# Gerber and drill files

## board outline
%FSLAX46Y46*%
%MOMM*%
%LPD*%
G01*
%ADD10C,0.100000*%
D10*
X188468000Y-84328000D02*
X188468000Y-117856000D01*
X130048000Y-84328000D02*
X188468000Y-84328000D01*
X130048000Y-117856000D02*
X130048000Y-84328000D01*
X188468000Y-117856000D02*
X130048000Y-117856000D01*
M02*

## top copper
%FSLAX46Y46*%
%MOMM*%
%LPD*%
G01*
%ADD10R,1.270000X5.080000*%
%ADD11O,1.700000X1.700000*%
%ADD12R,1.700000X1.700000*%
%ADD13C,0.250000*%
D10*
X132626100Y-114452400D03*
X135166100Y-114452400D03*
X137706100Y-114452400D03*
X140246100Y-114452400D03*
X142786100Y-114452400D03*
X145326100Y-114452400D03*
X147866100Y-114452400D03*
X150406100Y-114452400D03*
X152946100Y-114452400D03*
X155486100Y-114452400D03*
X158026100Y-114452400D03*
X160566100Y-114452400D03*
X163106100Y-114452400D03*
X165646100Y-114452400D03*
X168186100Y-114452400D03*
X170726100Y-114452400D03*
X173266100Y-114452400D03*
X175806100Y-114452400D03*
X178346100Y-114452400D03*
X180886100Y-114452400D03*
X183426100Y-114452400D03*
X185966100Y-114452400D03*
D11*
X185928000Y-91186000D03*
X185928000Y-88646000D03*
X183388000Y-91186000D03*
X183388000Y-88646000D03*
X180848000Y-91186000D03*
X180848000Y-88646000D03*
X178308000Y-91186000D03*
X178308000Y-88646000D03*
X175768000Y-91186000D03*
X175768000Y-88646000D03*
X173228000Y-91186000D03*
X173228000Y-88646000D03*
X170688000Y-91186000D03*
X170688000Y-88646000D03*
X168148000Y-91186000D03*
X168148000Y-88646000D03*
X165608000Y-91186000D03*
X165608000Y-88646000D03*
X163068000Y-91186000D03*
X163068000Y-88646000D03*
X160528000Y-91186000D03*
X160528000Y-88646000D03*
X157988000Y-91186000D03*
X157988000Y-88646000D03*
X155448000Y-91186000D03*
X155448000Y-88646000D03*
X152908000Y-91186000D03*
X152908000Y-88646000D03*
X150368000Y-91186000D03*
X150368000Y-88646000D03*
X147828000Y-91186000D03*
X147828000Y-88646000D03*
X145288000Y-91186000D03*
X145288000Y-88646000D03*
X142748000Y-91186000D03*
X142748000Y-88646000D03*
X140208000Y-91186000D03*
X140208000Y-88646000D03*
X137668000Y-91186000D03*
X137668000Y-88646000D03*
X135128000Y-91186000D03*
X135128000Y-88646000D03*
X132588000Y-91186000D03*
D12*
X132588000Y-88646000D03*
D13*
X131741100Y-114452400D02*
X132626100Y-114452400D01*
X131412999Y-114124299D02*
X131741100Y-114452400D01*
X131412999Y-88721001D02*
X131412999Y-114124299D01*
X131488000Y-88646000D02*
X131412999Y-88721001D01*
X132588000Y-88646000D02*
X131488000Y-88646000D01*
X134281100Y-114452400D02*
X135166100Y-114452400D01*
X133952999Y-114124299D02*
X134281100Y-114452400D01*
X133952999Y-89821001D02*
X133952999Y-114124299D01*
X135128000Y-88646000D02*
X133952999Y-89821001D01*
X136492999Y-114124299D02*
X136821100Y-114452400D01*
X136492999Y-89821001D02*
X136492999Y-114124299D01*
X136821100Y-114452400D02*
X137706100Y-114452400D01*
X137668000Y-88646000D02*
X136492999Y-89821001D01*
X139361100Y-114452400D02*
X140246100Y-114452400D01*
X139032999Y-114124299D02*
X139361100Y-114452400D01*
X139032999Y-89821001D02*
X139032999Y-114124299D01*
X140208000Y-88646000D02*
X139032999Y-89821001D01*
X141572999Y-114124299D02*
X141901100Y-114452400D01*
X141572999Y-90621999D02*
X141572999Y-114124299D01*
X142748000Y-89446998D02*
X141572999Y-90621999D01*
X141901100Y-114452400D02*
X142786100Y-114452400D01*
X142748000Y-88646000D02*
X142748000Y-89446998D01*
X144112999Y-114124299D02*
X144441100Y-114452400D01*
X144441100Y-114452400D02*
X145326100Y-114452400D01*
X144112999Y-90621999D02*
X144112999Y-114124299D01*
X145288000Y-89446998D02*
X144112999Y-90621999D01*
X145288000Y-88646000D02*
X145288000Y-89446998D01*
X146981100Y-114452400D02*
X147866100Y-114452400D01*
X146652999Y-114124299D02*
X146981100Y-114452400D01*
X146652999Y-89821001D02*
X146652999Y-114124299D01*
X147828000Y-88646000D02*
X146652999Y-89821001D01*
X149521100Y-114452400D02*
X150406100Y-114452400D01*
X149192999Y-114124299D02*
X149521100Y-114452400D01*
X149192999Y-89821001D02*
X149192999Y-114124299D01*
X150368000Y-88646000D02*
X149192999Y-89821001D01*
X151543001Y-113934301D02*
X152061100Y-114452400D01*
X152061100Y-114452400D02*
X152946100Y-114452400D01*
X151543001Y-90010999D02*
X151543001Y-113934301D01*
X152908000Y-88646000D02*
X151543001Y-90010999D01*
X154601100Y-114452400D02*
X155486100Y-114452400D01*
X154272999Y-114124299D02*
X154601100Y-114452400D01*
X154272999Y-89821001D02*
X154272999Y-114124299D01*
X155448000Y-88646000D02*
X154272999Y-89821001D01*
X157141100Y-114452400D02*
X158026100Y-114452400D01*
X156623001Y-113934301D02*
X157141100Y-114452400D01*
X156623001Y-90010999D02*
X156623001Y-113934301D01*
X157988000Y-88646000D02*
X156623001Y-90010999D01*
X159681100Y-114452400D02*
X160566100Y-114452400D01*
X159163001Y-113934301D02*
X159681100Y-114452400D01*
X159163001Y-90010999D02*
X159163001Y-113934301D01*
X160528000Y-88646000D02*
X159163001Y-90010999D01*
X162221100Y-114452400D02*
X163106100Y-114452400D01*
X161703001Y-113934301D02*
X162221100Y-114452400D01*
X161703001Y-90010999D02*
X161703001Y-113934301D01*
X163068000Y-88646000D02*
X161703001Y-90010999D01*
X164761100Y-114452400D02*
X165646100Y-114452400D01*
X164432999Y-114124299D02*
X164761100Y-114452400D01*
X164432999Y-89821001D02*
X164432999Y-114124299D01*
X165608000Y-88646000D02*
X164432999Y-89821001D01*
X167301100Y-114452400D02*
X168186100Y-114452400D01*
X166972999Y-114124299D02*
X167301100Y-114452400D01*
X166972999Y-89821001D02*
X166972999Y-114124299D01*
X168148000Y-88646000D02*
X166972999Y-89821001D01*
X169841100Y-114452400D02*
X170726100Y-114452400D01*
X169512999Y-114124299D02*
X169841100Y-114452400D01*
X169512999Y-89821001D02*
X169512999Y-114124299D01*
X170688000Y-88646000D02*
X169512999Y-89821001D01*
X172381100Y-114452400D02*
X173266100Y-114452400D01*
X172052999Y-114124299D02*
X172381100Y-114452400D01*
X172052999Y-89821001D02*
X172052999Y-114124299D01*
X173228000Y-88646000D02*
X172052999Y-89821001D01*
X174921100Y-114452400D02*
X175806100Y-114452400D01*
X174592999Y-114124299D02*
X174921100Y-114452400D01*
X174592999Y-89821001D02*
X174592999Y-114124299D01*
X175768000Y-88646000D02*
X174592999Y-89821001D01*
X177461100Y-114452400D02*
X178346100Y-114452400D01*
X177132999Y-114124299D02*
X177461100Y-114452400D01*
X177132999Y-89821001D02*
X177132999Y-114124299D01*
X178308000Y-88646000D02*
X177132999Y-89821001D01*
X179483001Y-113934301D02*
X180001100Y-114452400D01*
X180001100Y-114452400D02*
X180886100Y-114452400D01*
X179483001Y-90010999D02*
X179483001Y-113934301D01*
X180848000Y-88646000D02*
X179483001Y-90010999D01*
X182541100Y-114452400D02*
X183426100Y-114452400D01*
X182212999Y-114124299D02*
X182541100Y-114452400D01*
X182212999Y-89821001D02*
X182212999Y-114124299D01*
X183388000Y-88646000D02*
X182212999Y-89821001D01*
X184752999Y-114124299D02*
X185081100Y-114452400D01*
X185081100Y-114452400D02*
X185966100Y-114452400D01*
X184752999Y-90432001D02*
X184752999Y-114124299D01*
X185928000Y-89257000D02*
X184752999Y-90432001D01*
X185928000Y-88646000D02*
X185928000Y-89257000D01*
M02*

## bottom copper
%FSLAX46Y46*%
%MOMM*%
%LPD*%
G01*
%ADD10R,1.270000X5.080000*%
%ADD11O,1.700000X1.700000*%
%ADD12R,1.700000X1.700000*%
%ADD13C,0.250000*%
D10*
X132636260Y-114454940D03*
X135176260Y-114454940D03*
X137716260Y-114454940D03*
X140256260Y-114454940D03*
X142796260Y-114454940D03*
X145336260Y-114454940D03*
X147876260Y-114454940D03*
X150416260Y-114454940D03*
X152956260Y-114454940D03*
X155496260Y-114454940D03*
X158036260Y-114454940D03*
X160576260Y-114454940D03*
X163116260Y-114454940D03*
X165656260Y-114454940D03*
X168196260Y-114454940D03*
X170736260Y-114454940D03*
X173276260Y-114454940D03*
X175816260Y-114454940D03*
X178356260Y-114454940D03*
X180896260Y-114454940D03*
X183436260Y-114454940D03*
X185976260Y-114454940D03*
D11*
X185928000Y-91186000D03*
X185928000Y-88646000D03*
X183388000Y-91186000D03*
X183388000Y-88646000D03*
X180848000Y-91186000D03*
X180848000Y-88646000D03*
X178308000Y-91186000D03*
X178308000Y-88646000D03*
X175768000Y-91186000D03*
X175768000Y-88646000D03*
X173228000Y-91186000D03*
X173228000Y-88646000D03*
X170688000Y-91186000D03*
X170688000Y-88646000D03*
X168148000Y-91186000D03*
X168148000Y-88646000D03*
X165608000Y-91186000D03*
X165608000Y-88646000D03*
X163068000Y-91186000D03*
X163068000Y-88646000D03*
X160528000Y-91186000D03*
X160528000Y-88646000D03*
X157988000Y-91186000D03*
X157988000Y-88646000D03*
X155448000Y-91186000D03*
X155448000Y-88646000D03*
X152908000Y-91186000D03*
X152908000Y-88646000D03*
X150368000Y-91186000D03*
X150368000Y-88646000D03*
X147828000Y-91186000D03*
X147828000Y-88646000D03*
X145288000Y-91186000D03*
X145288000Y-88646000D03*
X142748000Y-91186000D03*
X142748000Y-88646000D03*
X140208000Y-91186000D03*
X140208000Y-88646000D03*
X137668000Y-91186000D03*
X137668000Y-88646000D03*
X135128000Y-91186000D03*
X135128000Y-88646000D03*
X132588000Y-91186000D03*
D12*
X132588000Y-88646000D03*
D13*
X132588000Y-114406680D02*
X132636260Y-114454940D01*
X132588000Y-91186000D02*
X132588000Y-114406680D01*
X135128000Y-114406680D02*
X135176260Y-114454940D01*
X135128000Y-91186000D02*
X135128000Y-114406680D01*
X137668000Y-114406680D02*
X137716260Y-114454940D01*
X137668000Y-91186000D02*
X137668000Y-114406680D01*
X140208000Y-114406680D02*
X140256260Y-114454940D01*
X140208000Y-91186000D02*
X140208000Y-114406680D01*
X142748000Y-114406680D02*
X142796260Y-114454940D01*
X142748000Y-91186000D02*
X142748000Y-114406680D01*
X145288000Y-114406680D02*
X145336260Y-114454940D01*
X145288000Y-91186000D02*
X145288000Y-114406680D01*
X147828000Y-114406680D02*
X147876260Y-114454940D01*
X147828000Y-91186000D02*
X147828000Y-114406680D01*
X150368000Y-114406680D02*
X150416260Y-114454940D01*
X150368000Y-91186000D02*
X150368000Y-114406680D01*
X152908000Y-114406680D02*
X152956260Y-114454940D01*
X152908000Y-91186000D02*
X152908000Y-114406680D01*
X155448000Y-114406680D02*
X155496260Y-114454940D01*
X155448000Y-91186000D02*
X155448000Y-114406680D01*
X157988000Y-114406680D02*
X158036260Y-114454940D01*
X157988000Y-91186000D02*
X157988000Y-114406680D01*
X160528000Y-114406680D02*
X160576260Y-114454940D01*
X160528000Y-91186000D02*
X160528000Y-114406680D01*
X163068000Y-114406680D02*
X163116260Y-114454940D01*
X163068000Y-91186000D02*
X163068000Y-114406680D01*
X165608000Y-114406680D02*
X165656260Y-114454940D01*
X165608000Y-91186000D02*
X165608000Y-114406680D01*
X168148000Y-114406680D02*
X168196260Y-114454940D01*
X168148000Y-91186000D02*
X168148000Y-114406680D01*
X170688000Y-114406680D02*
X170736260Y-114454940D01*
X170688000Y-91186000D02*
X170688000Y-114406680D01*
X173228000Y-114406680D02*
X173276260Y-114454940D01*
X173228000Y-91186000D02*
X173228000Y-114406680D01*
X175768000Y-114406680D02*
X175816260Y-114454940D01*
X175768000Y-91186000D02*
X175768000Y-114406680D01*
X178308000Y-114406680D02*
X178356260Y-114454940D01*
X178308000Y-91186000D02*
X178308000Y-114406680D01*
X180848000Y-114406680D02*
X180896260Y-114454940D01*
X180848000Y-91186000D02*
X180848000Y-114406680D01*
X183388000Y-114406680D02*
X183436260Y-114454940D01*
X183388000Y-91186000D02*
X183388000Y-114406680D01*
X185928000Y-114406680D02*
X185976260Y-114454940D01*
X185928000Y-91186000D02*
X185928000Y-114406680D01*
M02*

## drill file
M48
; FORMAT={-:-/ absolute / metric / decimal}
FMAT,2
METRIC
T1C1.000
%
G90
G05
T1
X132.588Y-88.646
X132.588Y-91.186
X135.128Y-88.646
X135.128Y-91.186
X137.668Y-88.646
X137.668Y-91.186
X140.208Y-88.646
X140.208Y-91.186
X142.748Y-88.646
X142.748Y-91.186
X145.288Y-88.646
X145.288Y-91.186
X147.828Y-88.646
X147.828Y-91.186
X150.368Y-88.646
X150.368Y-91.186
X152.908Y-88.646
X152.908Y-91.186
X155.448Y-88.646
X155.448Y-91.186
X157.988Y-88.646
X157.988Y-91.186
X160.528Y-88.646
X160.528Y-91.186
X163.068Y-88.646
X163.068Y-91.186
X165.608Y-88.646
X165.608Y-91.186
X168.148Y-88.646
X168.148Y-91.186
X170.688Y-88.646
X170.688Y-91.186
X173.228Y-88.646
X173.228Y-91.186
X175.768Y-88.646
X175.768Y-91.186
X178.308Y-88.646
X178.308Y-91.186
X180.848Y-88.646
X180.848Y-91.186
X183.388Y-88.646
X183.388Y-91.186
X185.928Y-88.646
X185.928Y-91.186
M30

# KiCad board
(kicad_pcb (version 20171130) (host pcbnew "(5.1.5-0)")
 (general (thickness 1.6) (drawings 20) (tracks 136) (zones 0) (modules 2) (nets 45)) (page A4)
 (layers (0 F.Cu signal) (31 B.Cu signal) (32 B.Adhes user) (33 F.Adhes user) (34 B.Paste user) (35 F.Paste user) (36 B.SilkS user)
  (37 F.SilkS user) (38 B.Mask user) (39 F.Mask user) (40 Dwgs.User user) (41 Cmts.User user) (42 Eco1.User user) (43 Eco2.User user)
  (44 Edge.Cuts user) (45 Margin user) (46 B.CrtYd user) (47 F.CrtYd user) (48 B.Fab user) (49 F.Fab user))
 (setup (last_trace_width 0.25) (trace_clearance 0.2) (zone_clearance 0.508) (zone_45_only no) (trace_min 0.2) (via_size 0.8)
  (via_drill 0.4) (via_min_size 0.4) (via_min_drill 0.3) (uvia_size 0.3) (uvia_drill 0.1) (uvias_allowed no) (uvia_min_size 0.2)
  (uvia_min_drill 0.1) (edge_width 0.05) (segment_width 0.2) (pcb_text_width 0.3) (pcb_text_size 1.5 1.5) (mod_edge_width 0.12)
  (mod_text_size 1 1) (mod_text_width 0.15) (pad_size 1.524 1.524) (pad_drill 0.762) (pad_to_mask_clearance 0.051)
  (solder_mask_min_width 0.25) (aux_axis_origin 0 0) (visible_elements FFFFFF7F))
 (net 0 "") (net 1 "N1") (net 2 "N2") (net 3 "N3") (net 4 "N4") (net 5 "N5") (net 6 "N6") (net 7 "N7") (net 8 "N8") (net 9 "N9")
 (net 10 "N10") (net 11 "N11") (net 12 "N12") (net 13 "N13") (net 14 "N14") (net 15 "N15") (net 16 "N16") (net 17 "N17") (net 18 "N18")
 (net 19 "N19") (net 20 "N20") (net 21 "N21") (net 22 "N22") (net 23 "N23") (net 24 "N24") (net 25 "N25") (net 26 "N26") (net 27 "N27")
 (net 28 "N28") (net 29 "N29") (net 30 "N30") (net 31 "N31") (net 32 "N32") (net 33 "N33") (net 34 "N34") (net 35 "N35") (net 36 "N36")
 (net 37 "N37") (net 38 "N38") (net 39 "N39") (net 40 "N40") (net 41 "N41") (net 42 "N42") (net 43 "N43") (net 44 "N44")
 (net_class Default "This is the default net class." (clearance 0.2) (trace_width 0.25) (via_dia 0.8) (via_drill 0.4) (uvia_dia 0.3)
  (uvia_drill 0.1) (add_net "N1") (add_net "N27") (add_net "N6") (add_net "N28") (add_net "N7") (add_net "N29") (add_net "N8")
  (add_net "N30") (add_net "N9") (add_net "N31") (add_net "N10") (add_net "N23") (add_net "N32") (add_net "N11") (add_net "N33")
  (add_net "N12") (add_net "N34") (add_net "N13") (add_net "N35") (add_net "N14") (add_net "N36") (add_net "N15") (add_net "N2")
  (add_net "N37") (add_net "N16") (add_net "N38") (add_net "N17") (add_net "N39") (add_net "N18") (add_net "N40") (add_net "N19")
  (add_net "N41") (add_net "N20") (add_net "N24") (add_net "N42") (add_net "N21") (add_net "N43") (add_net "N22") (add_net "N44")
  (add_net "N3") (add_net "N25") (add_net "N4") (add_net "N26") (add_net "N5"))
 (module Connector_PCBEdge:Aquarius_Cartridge (layer F.Cu) (at 144.272 102.362)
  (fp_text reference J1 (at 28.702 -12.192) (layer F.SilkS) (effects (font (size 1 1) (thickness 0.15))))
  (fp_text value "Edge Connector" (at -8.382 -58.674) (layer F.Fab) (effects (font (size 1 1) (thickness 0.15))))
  (pad 1 connect rect (at -11.6459 12.0904) (size 1.27 5.08) (layers F.Cu F.Mask) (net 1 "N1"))
  (pad 3 connect rect (at -9.1059 12.0904) (size 1.27 5.08) (layers F.Cu F.Mask) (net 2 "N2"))
  (pad 5 connect rect (at -6.5659 12.0904) (size 1.27 5.08) (layers F.Cu F.Mask) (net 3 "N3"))
  (pad 7 connect rect (at -4.0259 12.0904) (size 1.27 5.08) (layers F.Cu F.Mask) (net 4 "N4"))
  (pad 9 connect rect (at -1.4859 12.0904) (size 1.27 5.08) (layers F.Cu F.Mask) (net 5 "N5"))
  (pad 11 connect rect (at 1.0541 12.0904) (size 1.27 5.08) (layers F.Cu F.Mask) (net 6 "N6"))
  (pad 13 connect rect (at 3.5941 12.0904) (size 1.27 5.08) (layers F.Cu F.Mask) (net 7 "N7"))
  (pad 15 connect rect (at 6.1341 12.0904) (size 1.27 5.08) (layers F.Cu F.Mask) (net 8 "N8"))
  (pad 17 connect rect (at 8.6741 12.0904) (size 1.27 5.08) (layers F.Cu F.Mask) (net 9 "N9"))
  (pad 19 connect rect (at 11.2141 12.0904) (size 1.27 5.08) (layers F.Cu F.Mask) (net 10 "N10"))
  (pad 21 connect rect (at 13.7541 12.0904) (size 1.27 5.08) (layers F.Cu F.Mask) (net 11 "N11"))
  (pad 23 connect rect (at 16.2941 12.0904) (size 1.27 5.08) (layers F.Cu F.Mask) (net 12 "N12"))
  (pad 25 connect rect (at 18.8341 12.0904) (size 1.27 5.08) (layers F.Cu F.Mask) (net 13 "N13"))
  (pad 27 connect rect (at 21.3741 12.0904) (size 1.27 5.08) (layers F.Cu F.Mask) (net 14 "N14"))
  (pad 29 connect rect (at 23.9141 12.0904) (size 1.27 5.08) (layers F.Cu F.Mask) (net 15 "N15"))
  (pad 31 connect rect (at 26.4541 12.0904) (size 1.27 5.08) (layers F.Cu F.Mask) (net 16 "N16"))
  (pad 33 connect rect (at 28.9941 12.0904) (size 1.27 5.08) (layers F.Cu F.Mask) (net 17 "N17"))
  (pad 35 connect rect (at 31.5341 12.0904) (size 1.27 5.08) (layers F.Cu F.Mask) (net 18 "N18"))
  (pad 37 connect rect (at 34.0741 12.0904) (size 1.27 5.08) (layers F.Cu F.Mask) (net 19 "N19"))
  (pad 39 connect rect (at 36.6141 12.0904) (size 1.27 5.08) (layers F.Cu F.Mask) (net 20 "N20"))
  (pad 41 connect rect (at 39.1541 12.0904) (size 1.27 5.08) (layers F.Cu F.Mask) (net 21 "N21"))
  (pad 43 connect rect (at 41.6941 12.0904) (size 1.27 5.08) (layers F.Cu F.Mask) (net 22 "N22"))
  (pad 2 connect rect (at -11.63574 12.09294) (size 1.27 5.08) (layers B.Cu B.Mask) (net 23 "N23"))
  (pad 4 connect rect (at -9.09574 12.09294) (size 1.27 5.08) (layers B.Cu B.Mask) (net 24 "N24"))
  (pad 6 connect rect (at -6.55574 12.09294) (size 1.27 5.08) (layers B.Cu B.Mask) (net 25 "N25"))
  (pad 8 connect rect (at -4.01574 12.09294) (size 1.27 5.08) (layers B.Cu B.Mask) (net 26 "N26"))
  (pad 10 connect rect (at -1.47574 12.09294) (size 1.27 5.08) (layers B.Cu B.Mask) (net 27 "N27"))
  (pad 12 connect rect (at 1.06426 12.09294) (size 1.27 5.08) (layers B.Cu B.Mask) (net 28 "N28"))
  (pad 14 connect rect (at 3.60426 12.09294) (size 1.27 5.08) (layers B.Cu B.Mask) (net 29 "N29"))
  (pad 16 connect rect (at 6.14426 12.09294) (size 1.27 5.08) (layers B.Cu B.Mask) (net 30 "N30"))
  (pad 18 connect rect (at 8.68426 12.09294) (size 1.27 5.08) (layers B.Cu B.Mask) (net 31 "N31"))
  (pad 20 connect rect (at 11.22426 12.09294) (size 1.27 5.08) (layers B.Cu B.Mask) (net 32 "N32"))
  (pad 22 connect rect (at 13.76426 12.09294) (size 1.27 5.08) (layers B.Cu B.Mask) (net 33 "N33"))
  (pad 24 connect rect (at 16.30426 12.09294) (size 1.27 5.08) (layers B.Cu B.Mask) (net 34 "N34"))
  (pad 26 connect rect (at 18.84426 12.09294) (size 1.27 5.08) (layers B.Cu B.Mask) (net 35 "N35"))
  (pad 28 connect rect (at 21.38426 12.09294) (size 1.27 5.08) (layers B.Cu B.Mask) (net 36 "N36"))
  (pad 30 connect rect (at 23.92426 12.09294) (size 1.27 5.08) (layers B.Cu B.Mask) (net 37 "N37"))
  (pad 32 connect rect (at 26.46426 12.09294) (size 1.27 5.08) (layers B.Cu B.Mask) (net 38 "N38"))
  (pad 34 connect rect (at 29.00426 12.09294) (size 1.27 5.08) (layers B.Cu B.Mask) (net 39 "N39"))
  (pad 36 connect rect (at 31.54426 12.09294) (size 1.27 5.08) (layers B.Cu B.Mask) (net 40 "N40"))
  (pad 38 connect rect (at 34.08426 12.09294) (size 1.27 5.08) (layers B.Cu B.Mask) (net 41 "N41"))
  (pad 40 connect rect (at 36.62426 12.09294) (size 1.27 5.08) (layers B.Cu B.Mask) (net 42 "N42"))
  (pad 42 connect rect (at 39.16426 12.09294) (size 1.27 5.08) (layers B.Cu B.Mask) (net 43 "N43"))
  (pad 44 connect rect (at 41.70426 12.09294) (size 1.27 5.08) (layers B.Cu B.Mask) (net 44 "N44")))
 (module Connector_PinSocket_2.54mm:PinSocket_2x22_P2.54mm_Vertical (layer F.Cu) (at 132.588 88.646 90)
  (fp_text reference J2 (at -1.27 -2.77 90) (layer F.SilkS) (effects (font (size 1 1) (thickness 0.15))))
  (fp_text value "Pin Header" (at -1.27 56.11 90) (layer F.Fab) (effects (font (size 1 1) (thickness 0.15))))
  (pad 44 thru_hole oval (at -2.54 53.34 90) (size 1.7 1.7) (drill 1) (layers *.Cu *.Mask) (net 44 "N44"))
  (pad 43 thru_hole oval (at 0 53.34 90) (size 1.7 1.7) (drill 1) (layers *.Cu *.Mask) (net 22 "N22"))
  (pad 42 thru_hole oval (at -2.54 50.8 90) (size 1.7 1.7) (drill 1) (layers *.Cu *.Mask) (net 43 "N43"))
  (pad 41 thru_hole oval (at 0 50.8 90) (size 1.7 1.7) (drill 1) (layers *.Cu *.Mask) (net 21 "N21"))
  (pad 40 thru_hole oval (at -2.54 48.26 90) (size 1.7 1.7) (drill 1) (layers *.Cu *.Mask) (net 42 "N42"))
  (pad 39 thru_hole oval (at 0 48.26 90) (size 1.7 1.7) (drill 1) (layers *.Cu *.Mask) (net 20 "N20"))
  (pad 38 thru_hole oval (at -2.54 45.72 90) (size 1.7 1.7) (drill 1) (layers *.Cu *.Mask) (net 41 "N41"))
  (pad 37 thru_hole oval (at 0 45.72 90) (size 1.7 1.7) (drill 1) (layers *.Cu *.Mask) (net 19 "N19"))
  (pad 36 thru_hole oval (at -2.54 43.18 90) (size 1.7 1.7) (drill 1) (layers *.Cu *.Mask) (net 40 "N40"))
  (pad 35 thru_hole oval (at 0 43.18 90) (size 1.7 1.7) (drill 1) (layers *.Cu *.Mask) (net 18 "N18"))
  (pad 34 thru_hole oval (at -2.54 40.64 90) (size 1.7 1.7) (drill 1) (layers *.Cu *.Mask) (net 39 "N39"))
  (pad 33 thru_hole oval (at 0 40.64 90) (size 1.7 1.7) (drill 1) (layers *.Cu *.Mask) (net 17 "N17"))
  (pad 32 thru_hole oval (at -2.54 38.1 90) (size 1.7 1.7) (drill 1) (layers *.Cu *.Mask) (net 38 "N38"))
  (pad 31 thru_hole oval (at 0 38.1 90) (size 1.7 1.7) (drill 1) (layers *.Cu *.Mask) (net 16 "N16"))
  (pad 30 thru_hole oval (at -2.54 35.56 90) (size 1.7 1.7) (drill 1) (layers *.Cu *.Mask) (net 37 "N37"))
  (pad 29 thru_hole oval (at 0 35.56 90) (size 1.7 1.7) (drill 1) (layers *.Cu *.Mask) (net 15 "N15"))
  (pad 28 thru_hole oval (at -2.54 33.02 90) (size 1.7 1.7) (drill 1) (layers *.Cu *.Mask) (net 36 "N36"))
  (pad 27 thru_hole oval (at 0 33.02 90) (size 1.7 1.7) (drill 1) (layers *.Cu *.Mask) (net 14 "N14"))
  (pad 26 thru_hole oval (at -2.54 30.48 90) (size 1.7 1.7) (drill 1) (layers *.Cu *.Mask) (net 35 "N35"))
  (pad 25 thru_hole oval (at 0 30.48 90) (size 1.7 1.7) (drill 1) (layers *.Cu *.Mask) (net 13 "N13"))
  (pad 24 thru_hole oval (at -2.54 27.94 90) (size 1.7 1.7) (drill 1) (layers *.Cu *.Mask) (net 34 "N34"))
  (pad 23 thru_hole oval (at 0 27.94 90) (size 1.7 1.7) (drill 1) (layers *.Cu *.Mask) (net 12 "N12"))
  (pad 22 thru_hole oval (at -2.54 25.4 90) (size 1.7 1.7) (drill 1) (layers *.Cu *.Mask) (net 33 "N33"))
  (pad 21 thru_hole oval (at 0 25.4 90) (size 1.7 1.7) (drill 1) (layers *.Cu *.Mask) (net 11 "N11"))
  (pad 20 thru_hole oval (at -2.54 22.86 90) (size 1.7 1.7) (drill 1) (layers *.Cu *.Mask) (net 32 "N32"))
  (pad 19 thru_hole oval (at 0 22.86 90) (size 1.7 1.7) (drill 1) (layers *.Cu *.Mask) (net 10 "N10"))
  (pad 18 thru_hole oval (at -2.54 20.32 90) (size 1.7 1.7) (drill 1) (layers *.Cu *.Mask) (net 31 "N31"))
  (pad 17 thru_hole oval (at 0 20.32 90) (size 1.7 1.7) (drill 1) (layers *.Cu *.Mask) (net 9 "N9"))
  (pad 16 thru_hole oval (at -2.54 17.78 90) (size 1.7 1.7) (drill 1) (layers *.Cu *.Mask) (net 30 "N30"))
  (pad 15 thru_hole oval (at 0 17.78 90) (size 1.7 1.7) (drill 1) (layers *.Cu *.Mask) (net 8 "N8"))
  (pad 14 thru_hole oval (at -2.54 15.24 90) (size 1.7 1.7) (drill 1) (layers *.Cu *.Mask) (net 29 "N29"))
  (pad 13 thru_hole oval (at 0 15.24 90) (size 1.7 1.7) (drill 1) (layers *.Cu *.Mask) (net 7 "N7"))
  (pad 12 thru_hole oval (at -2.54 12.7 90) (size 1.7 1.7) (drill 1) (layers *.Cu *.Mask) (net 28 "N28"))
  (pad 11 thru_hole oval (at 0 12.7 90) (size 1.7 1.7) (drill 1) (layers *.Cu *.Mask) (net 6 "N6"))
  (pad 10 thru_hole oval (at -2.54 10.16 90) (size 1.7 1.7) (drill 1) (layers *.Cu *.Mask) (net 27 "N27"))
  (pad 9 thru_hole oval (at 0 10.16 90) (size 1.7 1.7) (drill 1) (layers *.Cu *.Mask) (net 5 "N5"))
  (pad 8 thru_hole oval (at -2.54 7.62 90) (size 1.7 1.7) (drill 1) (layers *.Cu *.Mask) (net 26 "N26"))
  (pad 7 thru_hole oval (at 0 7.62 90) (size 1.7 1.7) (drill 1) (layers *.Cu *.Mask) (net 4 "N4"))
  (pad 6 thru_hole oval (at -2.54 5.08 90) (size 1.7 1.7) (drill 1) (layers *.Cu *.Mask) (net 25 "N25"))
  (pad 5 thru_hole oval (at 0 5.08 90) (size 1.7 1.7) (drill 1) (layers *.Cu *.Mask) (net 3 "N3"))
  (pad 4 thru_hole oval (at -2.54 2.54 90) (size 1.7 1.7) (drill 1) (layers *.Cu *.Mask) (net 24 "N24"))
  (pad 3 thru_hole oval (at 0 2.54 90) (size 1.7 1.7) (drill 1) (layers *.Cu *.Mask) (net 2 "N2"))
  (pad 2 thru_hole oval (at -2.54 0 90) (size 1.7 1.7) (drill 1) (layers *.Cu *.Mask) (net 23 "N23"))
  (pad 1 thru_hole rect (at 0 0 90) (size 1.7 1.7) (drill 1) (layers *.Cu *.Mask) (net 1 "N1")))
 (gr_line (start 188.468 84.328) (end 188.468 117.856) (layer Edge.Cuts) (width 0.1))
 (gr_line (start 130.048 84.328) (end 188.468 84.328) (layer Edge.Cuts) (width 0.1))
 (gr_line (start 130.048 117.856) (end 130.048 84.328) (layer Edge.Cuts) (width 0.1))
 (gr_line (start 188.468 117.856) (end 130.048 117.856) (layer Edge.Cuts) (width 0.1))
 (segment (start 131.7411 114.4524) (end 132.6261 114.4524) (width 0.25) (layer F.Cu) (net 1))
 (segment (start 131.412999 114.124299) (end 131.7411 114.4524) (width 0.25) (layer F.Cu) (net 1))
 (segment (start 131.412999 88.721001) (end 131.412999 114.124299) (width 0.25) (layer F.Cu) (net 1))
 (segment (start 131.488 88.646) (end 131.412999 88.721001) (width 0.25) (layer F.Cu) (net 1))
 (segment (start 132.588 88.646) (end 131.488 88.646) (width 0.25) (layer F.Cu) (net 1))
 (segment (start 134.2811 114.4524) (end 135.1661 114.4524) (width 0.25) (layer F.Cu) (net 2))
 (segment (start 133.952999 114.124299) (end 134.2811 114.4524) (width 0.25) (layer F.Cu) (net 2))
 (segment (start 133.952999 89.821001) (end 133.952999 114.124299) (width 0.25) (layer F.Cu) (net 2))
 (segment (start 135.128 88.646) (end 133.952999 89.821001) (width 0.25) (layer F.Cu) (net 2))
 (segment (start 136.492999 114.124299) (end 136.8211 114.4524) (width 0.25) (layer F.Cu) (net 3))
 (segment (start 136.492999 89.821001) (end 136.492999 114.124299) (width 0.25) (layer F.Cu) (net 3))
 (segment (start 136.8211 114.4524) (end 137.7061 114.4524) (width 0.25) (layer F.Cu) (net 3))
 (segment (start 137.668 88.646) (end 136.492999 89.821001) (width 0.25) (layer F.Cu) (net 3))
 (segment (start 139.3611 114.4524) (end 140.2461 114.4524) (width 0.25) (layer F.Cu) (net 4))
 (segment (start 139.032999 114.124299) (end 139.3611 114.4524) (width 0.25) (layer F.Cu) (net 4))
 (segment (start 139.032999 89.821001) (end 139.032999 114.124299) (width 0.25) (layer F.Cu) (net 4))
 (segment (start 140.208 88.646) (end 139.032999 89.821001) (width 0.25) (layer F.Cu) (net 4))
 (segment (start 141.572999 114.124299) (end 141.9011 114.4524) (width 0.25) (layer F.Cu) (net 5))
 (segment (start 141.572999 90.621999) (end 141.572999 114.124299) (width 0.25) (layer F.Cu) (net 5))
 (segment (start 142.748 89.446998) (end 141.572999 90.621999) (width 0.25) (layer F.Cu) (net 5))
 (segment (start 141.9011 114.4524) (end 142.7861 114.4524) (width 0.25) (layer F.Cu) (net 5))
 (segment (start 142.748 88.646) (end 142.748 89.446998) (width 0.25) (layer F.Cu) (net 5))
 (segment (start 144.112999 114.124299) (end 144.4411 114.4524) (width 0.25) (layer F.Cu) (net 6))
 (segment (start 144.4411 114.4524) (end 145.3261 114.4524) (width 0.25) (layer F.Cu) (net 6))
 (segment (start 144.112999 90.621999) (end 144.112999 114.124299) (width 0.25) (layer F.Cu) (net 6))
 (segment (start 145.288 89.446998) (end 144.112999 90.621999) (width 0.25) (layer F.Cu) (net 6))
 (segment (start 145.288 88.646) (end 145.288 89.446998) (width 0.25) (layer F.Cu) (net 6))
 (segment (start 146.9811 114.4524) (end 147.8661 114.4524) (width 0.25) (layer F.Cu) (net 7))
 (segment (start 146.652999 114.124299) (end 146.9811 114.4524) (width 0.25) (layer F.Cu) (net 7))
 (segment (start 146.652999 89.821001) (end 146.652999 114.124299) (width 0.25) (layer F.Cu) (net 7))
 (segment (start 147.828 88.646) (end 146.652999 89.821001) (width 0.25) (layer F.Cu) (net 7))
 (segment (start 149.5211 114.4524) (end 150.4061 114.4524) (width 0.25) (layer F.Cu) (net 8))
 (segment (start 149.192999 114.124299) (end 149.5211 114.4524) (width 0.25) (layer F.Cu) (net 8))
 (segment (start 149.192999 89.821001) (end 149.192999 114.124299) (width 0.25) (layer F.Cu) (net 8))
 (segment (start 150.368 88.646) (end 149.192999 89.821001) (width 0.25) (layer F.Cu) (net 8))
 (segment (start 151.543001 113.934301) (end 152.0611 114.4524) (width 0.25) (layer F.Cu) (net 9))
 (segment (start 152.0611 114.4524) (end 152.9461 114.4524) (width 0.25) (layer F.Cu) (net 9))
 (segment (start 151.543001 90.010999) (end 151.543001 113.934301) (width 0.25) (layer F.Cu) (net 9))
 (segment (start 152.908 88.646) (end 151.543001 90.010999) (width 0.25) (layer F.Cu) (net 9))
 (segment (start 154.6011 114.4524) (end 155.4861 114.4524) (width 0.25) (layer F.Cu) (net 10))
 (segment (start 154.272999 114.124299) (end 154.6011 114.4524) (width 0.25) (layer F.Cu) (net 10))
 (segment (start 154.272999 89.821001) (end 154.272999 114.124299) (width 0.25) (layer F.Cu) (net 10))
 (segment (start 155.448 88.646) (end 154.272999 89.821001) (width 0.25) (layer F.Cu) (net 10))
 (segment (start 157.1411 114.4524) (end 158.0261 114.4524) (width 0.25) (layer F.Cu) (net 11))
 (segment (start 156.623001 113.934301) (end 157.1411 114.4524) (width 0.25) (layer F.Cu) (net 11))
 (segment (start 156.623001 90.010999) (end 156.623001 113.934301) (width 0.25) (layer F.Cu) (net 11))
 (segment (start 157.988 88.646) (end 156.623001 90.010999) (width 0.25) (layer F.Cu) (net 11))
 (segment (start 159.6811 114.4524) (end 160.5661 114.4524) (width 0.25) (layer F.Cu) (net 12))
 (segment (start 159.163001 113.934301) (end 159.6811 114.4524) (width 0.25) (layer F.Cu) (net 12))
 (segment (start 159.163001 90.010999) (end 159.163001 113.934301) (width 0.25) (layer F.Cu) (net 12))
 (segment (start 160.528 88.646) (end 159.163001 90.010999) (width 0.25) (layer F.Cu) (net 12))
 (segment (start 162.2211 114.4524) (end 163.1061 114.4524) (width 0.25) (layer F.Cu) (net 13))
 (segment (start 161.703001 113.934301) (end 162.2211 114.4524) (width 0.25) (layer F.Cu) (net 13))
 (segment (start 161.703001 90.010999) (end 161.703001 113.934301) (width 0.25) (layer F.Cu) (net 13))
 (segment (start 163.068 88.646) (end 161.703001 90.010999) (width 0.25) (layer F.Cu) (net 13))
 (segment (start 164.7611 114.4524) (end 165.6461 114.4524) (width 0.25) (layer F.Cu) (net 14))
 (segment (start 164.432999 114.124299) (end 164.7611 114.4524) (width 0.25) (layer F.Cu) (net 14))
 (segment (start 164.432999 89.821001) (end 164.432999 114.124299) (width 0.25) (layer F.Cu) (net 14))
 (segment (start 165.608 88.646) (end 164.432999 89.821001) (width 0.25) (layer F.Cu) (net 14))
 (segment (start 167.3011 114.4524) (end 168.1861 114.4524) (width 0.25) (layer F.Cu) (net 15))
 (segment (start 166.972999 114.124299) (end 167.3011 114.4524) (width 0.25) (layer F.Cu) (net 15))
 (segment (start 166.972999 89.821001) (end 166.972999 114.124299) (width 0.25) (layer F.Cu) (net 15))
 (segment (start 168.148 88.646) (end 166.972999 89.821001) (width 0.25) (layer F.Cu) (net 15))
 (segment (start 169.8411 114.4524) (end 170.7261 114.4524) (width 0.25) (layer F.Cu) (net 16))
 (segment (start 169.512999 114.124299) (end 169.8411 114.4524) (width 0.25) (layer F.Cu) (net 16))
 (segment (start 169.512999 89.821001) (end 169.512999 114.124299) (width 0.25) (layer F.Cu) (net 16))
 (segment (start 170.688 88.646) (end 169.512999 89.821001) (width 0.25) (layer F.Cu) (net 16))
 (segment (start 172.3811 114.4524) (end 173.2661 114.4524) (width 0.25) (layer F.Cu) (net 17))
 (segment (start 172.052999 114.124299) (end 172.3811 114.4524) (width 0.25) (layer F.Cu) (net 17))
 (segment (start 172.052999 89.821001) (end 172.052999 114.124299) (width 0.25) (layer F.Cu) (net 17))
 (segment (start 173.228 88.646) (end 172.052999 89.821001) (width 0.25) (layer F.Cu) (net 17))
 (segment (start 174.9211 114.4524) (end 175.8061 114.4524) (width 0.25) (layer F.Cu) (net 18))
 (segment (start 174.592999 114.124299) (end 174.9211 114.4524) (width 0.25) (layer F.Cu) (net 18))
 (segment (start 174.592999 89.821001) (end 174.592999 114.124299) (width 0.25) (layer F.Cu) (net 18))
 (segment (start 175.768 88.646) (end 174.592999 89.821001) (width 0.25) (layer F.Cu) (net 18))
 (segment (start 177.4611 114.4524) (end 178.3461 114.4524) (width 0.25) (layer F.Cu) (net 19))
 (segment (start 177.132999 114.124299) (end 177.4611 114.4524) (width 0.25) (layer F.Cu) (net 19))
 (segment (start 177.132999 89.821001) (end 177.132999 114.124299) (width 0.25) (layer F.Cu) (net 19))
 (segment (start 178.308 88.646) (end 177.132999 89.821001) (width 0.25) (layer F.Cu) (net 19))
 (segment (start 179.483001 113.934301) (end 180.0011 114.4524) (width 0.25) (layer F.Cu) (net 20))
 (segment (start 180.0011 114.4524) (end 180.8861 114.4524) (width 0.25) (layer F.Cu) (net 20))
 (segment (start 179.483001 90.010999) (end 179.483001 113.934301) (width 0.25) (layer F.Cu) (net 20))
 (segment (start 180.848 88.646) (end 179.483001 90.010999) (width 0.25) (layer F.Cu) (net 20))
 (segment (start 182.5411 114.4524) (end 183.4261 114.4524) (width 0.25) (layer F.Cu) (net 21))
 (segment (start 182.212999 114.124299) (end 182.5411 114.4524) (width 0.25) (layer F.Cu) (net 21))
 (segment (start 182.212999 89.821001) (end 182.212999 114.124299) (width 0.25) (layer F.Cu) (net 21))
 (segment (start 183.388 88.646) (end 182.212999 89.821001) (width 0.25) (layer F.Cu) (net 21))
 (segment (start 184.752999 114.124299) (end 185.0811 114.4524) (width 0.25) (layer F.Cu) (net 22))
 (segment (start 185.0811 114.4524) (end 185.9661 114.4524) (width 0.25) (layer F.Cu) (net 22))
 (segment (start 184.752999 90.432001) (end 184.752999 114.124299) (width 0.25) (layer F.Cu) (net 22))
 (segment (start 185.928 89.257) (end 184.752999 90.432001) (width 0.25) (layer F.Cu) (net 22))
 (segment (start 185.928 88.646) (end 185.928 89.257) (width 0.25) (layer F.Cu) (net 22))
 (segment (start 132.588 114.40668) (end 132.63626 114.45494) (width 0.25) (layer B.Cu) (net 23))
 (segment (start 132.588 91.186) (end 132.588 114.40668) (width 0.25) (layer B.Cu) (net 23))
 (segment (start 135.128 114.40668) (end 135.17626 114.45494) (width 0.25) (layer B.Cu) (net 24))
 (segment (start 135.128 91.186) (end 135.128 114.40668) (width 0.25) (layer B.Cu) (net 24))
 (segment (start 137.668 114.40668) (end 137.71626 114.45494) (width 0.25) (layer B.Cu) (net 25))
 (segment (start 137.668 91.186) (end 137.668 114.40668) (width 0.25) (layer B.Cu) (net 25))
 (segment (start 140.208 114.40668) (end 140.25626 114.45494) (width 0.25) (layer B.Cu) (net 26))
 (segment (start 140.208 91.186) (end 140.208 114.40668) (width 0.25) (layer B.Cu) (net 26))
 (segment (start 142.748 114.40668) (end 142.79626 114.45494) (width 0.25) (layer B.Cu) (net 27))
 (segment (start 142.748 91.186) (end 142.748 114.40668) (width 0.25) (layer B.Cu) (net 27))
 (segment (start 145.288 114.40668) (end 145.33626 114.45494) (width 0.25) (layer B.Cu) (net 28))
 (segment (start 145.288 91.186) (end 145.288 114.40668) (width 0.25) (layer B.Cu) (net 28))
 (segment (start 147.828 114.40668) (end 147.87626 114.45494) (width 0.25) (layer B.Cu) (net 29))
 (segment (start 147.828 91.186) (end 147.828 114.40668) (width 0.25) (layer B.Cu) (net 29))
 (segment (start 150.368 114.40668) (end 150.41626 114.45494) (width 0.25) (layer B.Cu) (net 30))
 (segment (start 150.368 91.186) (end 150.368 114.40668) (width 0.25) (layer B.Cu) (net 30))
 (segment (start 152.908 114.40668) (end 152.95626 114.45494) (width 0.25) (layer B.Cu) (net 31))
 (segment (start 152.908 91.186) (end 152.908 114.40668) (width 0.25) (layer B.Cu) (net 31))
 (segment (start 155.448 114.40668) (end 155.49626 114.45494) (width 0.25) (layer B.Cu) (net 32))
 (segment (start 155.448 91.186) (end 155.448 114.40668) (width 0.25) (layer B.Cu) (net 32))
 (segment (start 157.988 114.40668) (end 158.03626 114.45494) (width 0.25) (layer B.Cu) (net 33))
 (segment (start 157.988 91.186) (end 157.988 114.40668) (width 0.25) (layer B.Cu) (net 33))
 (segment (start 160.528 114.40668) (end 160.57626 114.45494) (width 0.25) (layer B.Cu) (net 34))
 (segment (start 160.528 91.186) (end 160.528 114.40668) (width 0.25) (layer B.Cu) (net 34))
 (segment (start 163.068 114.40668) (end 163.11626 114.45494) (width 0.25) (layer B.Cu) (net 35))
 (segment (start 163.068 91.186) (end 163.068 114.40668) (width 0.25) (layer B.Cu) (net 35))
 (segment (start 165.608 114.40668) (end 165.65626 114.45494) (width 0.25) (layer B.Cu) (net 36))
 (segment (start 165.608 91.186) (end 165.608 114.40668) (width 0.25) (layer B.Cu) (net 36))
 (segment (start 168.148 114.40668) (end 168.19626 114.45494) (width 0.25) (layer B.Cu) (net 37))
 (segment (start 168.148 91.186) (end 168.148 114.40668) (width 0.25) (layer B.Cu) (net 37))
 (segment (start 170.688 114.40668) (end 170.73626 114.45494) (width 0.25) (layer B.Cu) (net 38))
 (segment (start 170.688 91.186) (end 170.688 114.40668) (width 0.25) (layer B.Cu) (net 38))
 (segment (start 173.228 114.40668) (end 173.27626 114.45494) (width 0.25) (layer B.Cu) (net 39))
 (segment (start 173.228 91.186) (end 173.228 114.40668) (width 0.25) (layer B.Cu) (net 39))
 (segment (start 175.768 114.40668) (end 175.81626 114.45494) (width 0.25) (layer B.Cu) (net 40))
 (segment (start 175.768 91.186) (end 175.768 114.40668) (width 0.25) (layer B.Cu) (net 40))
 (segment (start 178.308 114.40668) (end 178.35626 114.45494) (width 0.25) (layer B.Cu) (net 41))
 (segment (start 178.308 91.186) (end 178.308 114.40668) (width 0.25) (layer B.Cu) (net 41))
 (segment (start 180.848 114.40668) (end 180.89626 114.45494) (width 0.25) (layer B.Cu) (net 42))
 (segment (start 180.848 91.186) (end 180.848 114.40668) (width 0.25) (layer B.Cu) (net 42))
 (segment (start 183.388 114.40668) (end 183.43626 114.45494) (width 0.25) (layer B.Cu) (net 43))
 (segment (start 183.388 91.186) (end 183.388 114.40668) (width 0.25) (layer B.Cu) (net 43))
 (segment (start 185.928 114.40668) (end 185.97626 114.45494) (width 0.25) (layer B.Cu) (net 44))
 (segment (start 185.928 91.186) (end 185.928 114.40668) (width 0.25) (layer B.Cu) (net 44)))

